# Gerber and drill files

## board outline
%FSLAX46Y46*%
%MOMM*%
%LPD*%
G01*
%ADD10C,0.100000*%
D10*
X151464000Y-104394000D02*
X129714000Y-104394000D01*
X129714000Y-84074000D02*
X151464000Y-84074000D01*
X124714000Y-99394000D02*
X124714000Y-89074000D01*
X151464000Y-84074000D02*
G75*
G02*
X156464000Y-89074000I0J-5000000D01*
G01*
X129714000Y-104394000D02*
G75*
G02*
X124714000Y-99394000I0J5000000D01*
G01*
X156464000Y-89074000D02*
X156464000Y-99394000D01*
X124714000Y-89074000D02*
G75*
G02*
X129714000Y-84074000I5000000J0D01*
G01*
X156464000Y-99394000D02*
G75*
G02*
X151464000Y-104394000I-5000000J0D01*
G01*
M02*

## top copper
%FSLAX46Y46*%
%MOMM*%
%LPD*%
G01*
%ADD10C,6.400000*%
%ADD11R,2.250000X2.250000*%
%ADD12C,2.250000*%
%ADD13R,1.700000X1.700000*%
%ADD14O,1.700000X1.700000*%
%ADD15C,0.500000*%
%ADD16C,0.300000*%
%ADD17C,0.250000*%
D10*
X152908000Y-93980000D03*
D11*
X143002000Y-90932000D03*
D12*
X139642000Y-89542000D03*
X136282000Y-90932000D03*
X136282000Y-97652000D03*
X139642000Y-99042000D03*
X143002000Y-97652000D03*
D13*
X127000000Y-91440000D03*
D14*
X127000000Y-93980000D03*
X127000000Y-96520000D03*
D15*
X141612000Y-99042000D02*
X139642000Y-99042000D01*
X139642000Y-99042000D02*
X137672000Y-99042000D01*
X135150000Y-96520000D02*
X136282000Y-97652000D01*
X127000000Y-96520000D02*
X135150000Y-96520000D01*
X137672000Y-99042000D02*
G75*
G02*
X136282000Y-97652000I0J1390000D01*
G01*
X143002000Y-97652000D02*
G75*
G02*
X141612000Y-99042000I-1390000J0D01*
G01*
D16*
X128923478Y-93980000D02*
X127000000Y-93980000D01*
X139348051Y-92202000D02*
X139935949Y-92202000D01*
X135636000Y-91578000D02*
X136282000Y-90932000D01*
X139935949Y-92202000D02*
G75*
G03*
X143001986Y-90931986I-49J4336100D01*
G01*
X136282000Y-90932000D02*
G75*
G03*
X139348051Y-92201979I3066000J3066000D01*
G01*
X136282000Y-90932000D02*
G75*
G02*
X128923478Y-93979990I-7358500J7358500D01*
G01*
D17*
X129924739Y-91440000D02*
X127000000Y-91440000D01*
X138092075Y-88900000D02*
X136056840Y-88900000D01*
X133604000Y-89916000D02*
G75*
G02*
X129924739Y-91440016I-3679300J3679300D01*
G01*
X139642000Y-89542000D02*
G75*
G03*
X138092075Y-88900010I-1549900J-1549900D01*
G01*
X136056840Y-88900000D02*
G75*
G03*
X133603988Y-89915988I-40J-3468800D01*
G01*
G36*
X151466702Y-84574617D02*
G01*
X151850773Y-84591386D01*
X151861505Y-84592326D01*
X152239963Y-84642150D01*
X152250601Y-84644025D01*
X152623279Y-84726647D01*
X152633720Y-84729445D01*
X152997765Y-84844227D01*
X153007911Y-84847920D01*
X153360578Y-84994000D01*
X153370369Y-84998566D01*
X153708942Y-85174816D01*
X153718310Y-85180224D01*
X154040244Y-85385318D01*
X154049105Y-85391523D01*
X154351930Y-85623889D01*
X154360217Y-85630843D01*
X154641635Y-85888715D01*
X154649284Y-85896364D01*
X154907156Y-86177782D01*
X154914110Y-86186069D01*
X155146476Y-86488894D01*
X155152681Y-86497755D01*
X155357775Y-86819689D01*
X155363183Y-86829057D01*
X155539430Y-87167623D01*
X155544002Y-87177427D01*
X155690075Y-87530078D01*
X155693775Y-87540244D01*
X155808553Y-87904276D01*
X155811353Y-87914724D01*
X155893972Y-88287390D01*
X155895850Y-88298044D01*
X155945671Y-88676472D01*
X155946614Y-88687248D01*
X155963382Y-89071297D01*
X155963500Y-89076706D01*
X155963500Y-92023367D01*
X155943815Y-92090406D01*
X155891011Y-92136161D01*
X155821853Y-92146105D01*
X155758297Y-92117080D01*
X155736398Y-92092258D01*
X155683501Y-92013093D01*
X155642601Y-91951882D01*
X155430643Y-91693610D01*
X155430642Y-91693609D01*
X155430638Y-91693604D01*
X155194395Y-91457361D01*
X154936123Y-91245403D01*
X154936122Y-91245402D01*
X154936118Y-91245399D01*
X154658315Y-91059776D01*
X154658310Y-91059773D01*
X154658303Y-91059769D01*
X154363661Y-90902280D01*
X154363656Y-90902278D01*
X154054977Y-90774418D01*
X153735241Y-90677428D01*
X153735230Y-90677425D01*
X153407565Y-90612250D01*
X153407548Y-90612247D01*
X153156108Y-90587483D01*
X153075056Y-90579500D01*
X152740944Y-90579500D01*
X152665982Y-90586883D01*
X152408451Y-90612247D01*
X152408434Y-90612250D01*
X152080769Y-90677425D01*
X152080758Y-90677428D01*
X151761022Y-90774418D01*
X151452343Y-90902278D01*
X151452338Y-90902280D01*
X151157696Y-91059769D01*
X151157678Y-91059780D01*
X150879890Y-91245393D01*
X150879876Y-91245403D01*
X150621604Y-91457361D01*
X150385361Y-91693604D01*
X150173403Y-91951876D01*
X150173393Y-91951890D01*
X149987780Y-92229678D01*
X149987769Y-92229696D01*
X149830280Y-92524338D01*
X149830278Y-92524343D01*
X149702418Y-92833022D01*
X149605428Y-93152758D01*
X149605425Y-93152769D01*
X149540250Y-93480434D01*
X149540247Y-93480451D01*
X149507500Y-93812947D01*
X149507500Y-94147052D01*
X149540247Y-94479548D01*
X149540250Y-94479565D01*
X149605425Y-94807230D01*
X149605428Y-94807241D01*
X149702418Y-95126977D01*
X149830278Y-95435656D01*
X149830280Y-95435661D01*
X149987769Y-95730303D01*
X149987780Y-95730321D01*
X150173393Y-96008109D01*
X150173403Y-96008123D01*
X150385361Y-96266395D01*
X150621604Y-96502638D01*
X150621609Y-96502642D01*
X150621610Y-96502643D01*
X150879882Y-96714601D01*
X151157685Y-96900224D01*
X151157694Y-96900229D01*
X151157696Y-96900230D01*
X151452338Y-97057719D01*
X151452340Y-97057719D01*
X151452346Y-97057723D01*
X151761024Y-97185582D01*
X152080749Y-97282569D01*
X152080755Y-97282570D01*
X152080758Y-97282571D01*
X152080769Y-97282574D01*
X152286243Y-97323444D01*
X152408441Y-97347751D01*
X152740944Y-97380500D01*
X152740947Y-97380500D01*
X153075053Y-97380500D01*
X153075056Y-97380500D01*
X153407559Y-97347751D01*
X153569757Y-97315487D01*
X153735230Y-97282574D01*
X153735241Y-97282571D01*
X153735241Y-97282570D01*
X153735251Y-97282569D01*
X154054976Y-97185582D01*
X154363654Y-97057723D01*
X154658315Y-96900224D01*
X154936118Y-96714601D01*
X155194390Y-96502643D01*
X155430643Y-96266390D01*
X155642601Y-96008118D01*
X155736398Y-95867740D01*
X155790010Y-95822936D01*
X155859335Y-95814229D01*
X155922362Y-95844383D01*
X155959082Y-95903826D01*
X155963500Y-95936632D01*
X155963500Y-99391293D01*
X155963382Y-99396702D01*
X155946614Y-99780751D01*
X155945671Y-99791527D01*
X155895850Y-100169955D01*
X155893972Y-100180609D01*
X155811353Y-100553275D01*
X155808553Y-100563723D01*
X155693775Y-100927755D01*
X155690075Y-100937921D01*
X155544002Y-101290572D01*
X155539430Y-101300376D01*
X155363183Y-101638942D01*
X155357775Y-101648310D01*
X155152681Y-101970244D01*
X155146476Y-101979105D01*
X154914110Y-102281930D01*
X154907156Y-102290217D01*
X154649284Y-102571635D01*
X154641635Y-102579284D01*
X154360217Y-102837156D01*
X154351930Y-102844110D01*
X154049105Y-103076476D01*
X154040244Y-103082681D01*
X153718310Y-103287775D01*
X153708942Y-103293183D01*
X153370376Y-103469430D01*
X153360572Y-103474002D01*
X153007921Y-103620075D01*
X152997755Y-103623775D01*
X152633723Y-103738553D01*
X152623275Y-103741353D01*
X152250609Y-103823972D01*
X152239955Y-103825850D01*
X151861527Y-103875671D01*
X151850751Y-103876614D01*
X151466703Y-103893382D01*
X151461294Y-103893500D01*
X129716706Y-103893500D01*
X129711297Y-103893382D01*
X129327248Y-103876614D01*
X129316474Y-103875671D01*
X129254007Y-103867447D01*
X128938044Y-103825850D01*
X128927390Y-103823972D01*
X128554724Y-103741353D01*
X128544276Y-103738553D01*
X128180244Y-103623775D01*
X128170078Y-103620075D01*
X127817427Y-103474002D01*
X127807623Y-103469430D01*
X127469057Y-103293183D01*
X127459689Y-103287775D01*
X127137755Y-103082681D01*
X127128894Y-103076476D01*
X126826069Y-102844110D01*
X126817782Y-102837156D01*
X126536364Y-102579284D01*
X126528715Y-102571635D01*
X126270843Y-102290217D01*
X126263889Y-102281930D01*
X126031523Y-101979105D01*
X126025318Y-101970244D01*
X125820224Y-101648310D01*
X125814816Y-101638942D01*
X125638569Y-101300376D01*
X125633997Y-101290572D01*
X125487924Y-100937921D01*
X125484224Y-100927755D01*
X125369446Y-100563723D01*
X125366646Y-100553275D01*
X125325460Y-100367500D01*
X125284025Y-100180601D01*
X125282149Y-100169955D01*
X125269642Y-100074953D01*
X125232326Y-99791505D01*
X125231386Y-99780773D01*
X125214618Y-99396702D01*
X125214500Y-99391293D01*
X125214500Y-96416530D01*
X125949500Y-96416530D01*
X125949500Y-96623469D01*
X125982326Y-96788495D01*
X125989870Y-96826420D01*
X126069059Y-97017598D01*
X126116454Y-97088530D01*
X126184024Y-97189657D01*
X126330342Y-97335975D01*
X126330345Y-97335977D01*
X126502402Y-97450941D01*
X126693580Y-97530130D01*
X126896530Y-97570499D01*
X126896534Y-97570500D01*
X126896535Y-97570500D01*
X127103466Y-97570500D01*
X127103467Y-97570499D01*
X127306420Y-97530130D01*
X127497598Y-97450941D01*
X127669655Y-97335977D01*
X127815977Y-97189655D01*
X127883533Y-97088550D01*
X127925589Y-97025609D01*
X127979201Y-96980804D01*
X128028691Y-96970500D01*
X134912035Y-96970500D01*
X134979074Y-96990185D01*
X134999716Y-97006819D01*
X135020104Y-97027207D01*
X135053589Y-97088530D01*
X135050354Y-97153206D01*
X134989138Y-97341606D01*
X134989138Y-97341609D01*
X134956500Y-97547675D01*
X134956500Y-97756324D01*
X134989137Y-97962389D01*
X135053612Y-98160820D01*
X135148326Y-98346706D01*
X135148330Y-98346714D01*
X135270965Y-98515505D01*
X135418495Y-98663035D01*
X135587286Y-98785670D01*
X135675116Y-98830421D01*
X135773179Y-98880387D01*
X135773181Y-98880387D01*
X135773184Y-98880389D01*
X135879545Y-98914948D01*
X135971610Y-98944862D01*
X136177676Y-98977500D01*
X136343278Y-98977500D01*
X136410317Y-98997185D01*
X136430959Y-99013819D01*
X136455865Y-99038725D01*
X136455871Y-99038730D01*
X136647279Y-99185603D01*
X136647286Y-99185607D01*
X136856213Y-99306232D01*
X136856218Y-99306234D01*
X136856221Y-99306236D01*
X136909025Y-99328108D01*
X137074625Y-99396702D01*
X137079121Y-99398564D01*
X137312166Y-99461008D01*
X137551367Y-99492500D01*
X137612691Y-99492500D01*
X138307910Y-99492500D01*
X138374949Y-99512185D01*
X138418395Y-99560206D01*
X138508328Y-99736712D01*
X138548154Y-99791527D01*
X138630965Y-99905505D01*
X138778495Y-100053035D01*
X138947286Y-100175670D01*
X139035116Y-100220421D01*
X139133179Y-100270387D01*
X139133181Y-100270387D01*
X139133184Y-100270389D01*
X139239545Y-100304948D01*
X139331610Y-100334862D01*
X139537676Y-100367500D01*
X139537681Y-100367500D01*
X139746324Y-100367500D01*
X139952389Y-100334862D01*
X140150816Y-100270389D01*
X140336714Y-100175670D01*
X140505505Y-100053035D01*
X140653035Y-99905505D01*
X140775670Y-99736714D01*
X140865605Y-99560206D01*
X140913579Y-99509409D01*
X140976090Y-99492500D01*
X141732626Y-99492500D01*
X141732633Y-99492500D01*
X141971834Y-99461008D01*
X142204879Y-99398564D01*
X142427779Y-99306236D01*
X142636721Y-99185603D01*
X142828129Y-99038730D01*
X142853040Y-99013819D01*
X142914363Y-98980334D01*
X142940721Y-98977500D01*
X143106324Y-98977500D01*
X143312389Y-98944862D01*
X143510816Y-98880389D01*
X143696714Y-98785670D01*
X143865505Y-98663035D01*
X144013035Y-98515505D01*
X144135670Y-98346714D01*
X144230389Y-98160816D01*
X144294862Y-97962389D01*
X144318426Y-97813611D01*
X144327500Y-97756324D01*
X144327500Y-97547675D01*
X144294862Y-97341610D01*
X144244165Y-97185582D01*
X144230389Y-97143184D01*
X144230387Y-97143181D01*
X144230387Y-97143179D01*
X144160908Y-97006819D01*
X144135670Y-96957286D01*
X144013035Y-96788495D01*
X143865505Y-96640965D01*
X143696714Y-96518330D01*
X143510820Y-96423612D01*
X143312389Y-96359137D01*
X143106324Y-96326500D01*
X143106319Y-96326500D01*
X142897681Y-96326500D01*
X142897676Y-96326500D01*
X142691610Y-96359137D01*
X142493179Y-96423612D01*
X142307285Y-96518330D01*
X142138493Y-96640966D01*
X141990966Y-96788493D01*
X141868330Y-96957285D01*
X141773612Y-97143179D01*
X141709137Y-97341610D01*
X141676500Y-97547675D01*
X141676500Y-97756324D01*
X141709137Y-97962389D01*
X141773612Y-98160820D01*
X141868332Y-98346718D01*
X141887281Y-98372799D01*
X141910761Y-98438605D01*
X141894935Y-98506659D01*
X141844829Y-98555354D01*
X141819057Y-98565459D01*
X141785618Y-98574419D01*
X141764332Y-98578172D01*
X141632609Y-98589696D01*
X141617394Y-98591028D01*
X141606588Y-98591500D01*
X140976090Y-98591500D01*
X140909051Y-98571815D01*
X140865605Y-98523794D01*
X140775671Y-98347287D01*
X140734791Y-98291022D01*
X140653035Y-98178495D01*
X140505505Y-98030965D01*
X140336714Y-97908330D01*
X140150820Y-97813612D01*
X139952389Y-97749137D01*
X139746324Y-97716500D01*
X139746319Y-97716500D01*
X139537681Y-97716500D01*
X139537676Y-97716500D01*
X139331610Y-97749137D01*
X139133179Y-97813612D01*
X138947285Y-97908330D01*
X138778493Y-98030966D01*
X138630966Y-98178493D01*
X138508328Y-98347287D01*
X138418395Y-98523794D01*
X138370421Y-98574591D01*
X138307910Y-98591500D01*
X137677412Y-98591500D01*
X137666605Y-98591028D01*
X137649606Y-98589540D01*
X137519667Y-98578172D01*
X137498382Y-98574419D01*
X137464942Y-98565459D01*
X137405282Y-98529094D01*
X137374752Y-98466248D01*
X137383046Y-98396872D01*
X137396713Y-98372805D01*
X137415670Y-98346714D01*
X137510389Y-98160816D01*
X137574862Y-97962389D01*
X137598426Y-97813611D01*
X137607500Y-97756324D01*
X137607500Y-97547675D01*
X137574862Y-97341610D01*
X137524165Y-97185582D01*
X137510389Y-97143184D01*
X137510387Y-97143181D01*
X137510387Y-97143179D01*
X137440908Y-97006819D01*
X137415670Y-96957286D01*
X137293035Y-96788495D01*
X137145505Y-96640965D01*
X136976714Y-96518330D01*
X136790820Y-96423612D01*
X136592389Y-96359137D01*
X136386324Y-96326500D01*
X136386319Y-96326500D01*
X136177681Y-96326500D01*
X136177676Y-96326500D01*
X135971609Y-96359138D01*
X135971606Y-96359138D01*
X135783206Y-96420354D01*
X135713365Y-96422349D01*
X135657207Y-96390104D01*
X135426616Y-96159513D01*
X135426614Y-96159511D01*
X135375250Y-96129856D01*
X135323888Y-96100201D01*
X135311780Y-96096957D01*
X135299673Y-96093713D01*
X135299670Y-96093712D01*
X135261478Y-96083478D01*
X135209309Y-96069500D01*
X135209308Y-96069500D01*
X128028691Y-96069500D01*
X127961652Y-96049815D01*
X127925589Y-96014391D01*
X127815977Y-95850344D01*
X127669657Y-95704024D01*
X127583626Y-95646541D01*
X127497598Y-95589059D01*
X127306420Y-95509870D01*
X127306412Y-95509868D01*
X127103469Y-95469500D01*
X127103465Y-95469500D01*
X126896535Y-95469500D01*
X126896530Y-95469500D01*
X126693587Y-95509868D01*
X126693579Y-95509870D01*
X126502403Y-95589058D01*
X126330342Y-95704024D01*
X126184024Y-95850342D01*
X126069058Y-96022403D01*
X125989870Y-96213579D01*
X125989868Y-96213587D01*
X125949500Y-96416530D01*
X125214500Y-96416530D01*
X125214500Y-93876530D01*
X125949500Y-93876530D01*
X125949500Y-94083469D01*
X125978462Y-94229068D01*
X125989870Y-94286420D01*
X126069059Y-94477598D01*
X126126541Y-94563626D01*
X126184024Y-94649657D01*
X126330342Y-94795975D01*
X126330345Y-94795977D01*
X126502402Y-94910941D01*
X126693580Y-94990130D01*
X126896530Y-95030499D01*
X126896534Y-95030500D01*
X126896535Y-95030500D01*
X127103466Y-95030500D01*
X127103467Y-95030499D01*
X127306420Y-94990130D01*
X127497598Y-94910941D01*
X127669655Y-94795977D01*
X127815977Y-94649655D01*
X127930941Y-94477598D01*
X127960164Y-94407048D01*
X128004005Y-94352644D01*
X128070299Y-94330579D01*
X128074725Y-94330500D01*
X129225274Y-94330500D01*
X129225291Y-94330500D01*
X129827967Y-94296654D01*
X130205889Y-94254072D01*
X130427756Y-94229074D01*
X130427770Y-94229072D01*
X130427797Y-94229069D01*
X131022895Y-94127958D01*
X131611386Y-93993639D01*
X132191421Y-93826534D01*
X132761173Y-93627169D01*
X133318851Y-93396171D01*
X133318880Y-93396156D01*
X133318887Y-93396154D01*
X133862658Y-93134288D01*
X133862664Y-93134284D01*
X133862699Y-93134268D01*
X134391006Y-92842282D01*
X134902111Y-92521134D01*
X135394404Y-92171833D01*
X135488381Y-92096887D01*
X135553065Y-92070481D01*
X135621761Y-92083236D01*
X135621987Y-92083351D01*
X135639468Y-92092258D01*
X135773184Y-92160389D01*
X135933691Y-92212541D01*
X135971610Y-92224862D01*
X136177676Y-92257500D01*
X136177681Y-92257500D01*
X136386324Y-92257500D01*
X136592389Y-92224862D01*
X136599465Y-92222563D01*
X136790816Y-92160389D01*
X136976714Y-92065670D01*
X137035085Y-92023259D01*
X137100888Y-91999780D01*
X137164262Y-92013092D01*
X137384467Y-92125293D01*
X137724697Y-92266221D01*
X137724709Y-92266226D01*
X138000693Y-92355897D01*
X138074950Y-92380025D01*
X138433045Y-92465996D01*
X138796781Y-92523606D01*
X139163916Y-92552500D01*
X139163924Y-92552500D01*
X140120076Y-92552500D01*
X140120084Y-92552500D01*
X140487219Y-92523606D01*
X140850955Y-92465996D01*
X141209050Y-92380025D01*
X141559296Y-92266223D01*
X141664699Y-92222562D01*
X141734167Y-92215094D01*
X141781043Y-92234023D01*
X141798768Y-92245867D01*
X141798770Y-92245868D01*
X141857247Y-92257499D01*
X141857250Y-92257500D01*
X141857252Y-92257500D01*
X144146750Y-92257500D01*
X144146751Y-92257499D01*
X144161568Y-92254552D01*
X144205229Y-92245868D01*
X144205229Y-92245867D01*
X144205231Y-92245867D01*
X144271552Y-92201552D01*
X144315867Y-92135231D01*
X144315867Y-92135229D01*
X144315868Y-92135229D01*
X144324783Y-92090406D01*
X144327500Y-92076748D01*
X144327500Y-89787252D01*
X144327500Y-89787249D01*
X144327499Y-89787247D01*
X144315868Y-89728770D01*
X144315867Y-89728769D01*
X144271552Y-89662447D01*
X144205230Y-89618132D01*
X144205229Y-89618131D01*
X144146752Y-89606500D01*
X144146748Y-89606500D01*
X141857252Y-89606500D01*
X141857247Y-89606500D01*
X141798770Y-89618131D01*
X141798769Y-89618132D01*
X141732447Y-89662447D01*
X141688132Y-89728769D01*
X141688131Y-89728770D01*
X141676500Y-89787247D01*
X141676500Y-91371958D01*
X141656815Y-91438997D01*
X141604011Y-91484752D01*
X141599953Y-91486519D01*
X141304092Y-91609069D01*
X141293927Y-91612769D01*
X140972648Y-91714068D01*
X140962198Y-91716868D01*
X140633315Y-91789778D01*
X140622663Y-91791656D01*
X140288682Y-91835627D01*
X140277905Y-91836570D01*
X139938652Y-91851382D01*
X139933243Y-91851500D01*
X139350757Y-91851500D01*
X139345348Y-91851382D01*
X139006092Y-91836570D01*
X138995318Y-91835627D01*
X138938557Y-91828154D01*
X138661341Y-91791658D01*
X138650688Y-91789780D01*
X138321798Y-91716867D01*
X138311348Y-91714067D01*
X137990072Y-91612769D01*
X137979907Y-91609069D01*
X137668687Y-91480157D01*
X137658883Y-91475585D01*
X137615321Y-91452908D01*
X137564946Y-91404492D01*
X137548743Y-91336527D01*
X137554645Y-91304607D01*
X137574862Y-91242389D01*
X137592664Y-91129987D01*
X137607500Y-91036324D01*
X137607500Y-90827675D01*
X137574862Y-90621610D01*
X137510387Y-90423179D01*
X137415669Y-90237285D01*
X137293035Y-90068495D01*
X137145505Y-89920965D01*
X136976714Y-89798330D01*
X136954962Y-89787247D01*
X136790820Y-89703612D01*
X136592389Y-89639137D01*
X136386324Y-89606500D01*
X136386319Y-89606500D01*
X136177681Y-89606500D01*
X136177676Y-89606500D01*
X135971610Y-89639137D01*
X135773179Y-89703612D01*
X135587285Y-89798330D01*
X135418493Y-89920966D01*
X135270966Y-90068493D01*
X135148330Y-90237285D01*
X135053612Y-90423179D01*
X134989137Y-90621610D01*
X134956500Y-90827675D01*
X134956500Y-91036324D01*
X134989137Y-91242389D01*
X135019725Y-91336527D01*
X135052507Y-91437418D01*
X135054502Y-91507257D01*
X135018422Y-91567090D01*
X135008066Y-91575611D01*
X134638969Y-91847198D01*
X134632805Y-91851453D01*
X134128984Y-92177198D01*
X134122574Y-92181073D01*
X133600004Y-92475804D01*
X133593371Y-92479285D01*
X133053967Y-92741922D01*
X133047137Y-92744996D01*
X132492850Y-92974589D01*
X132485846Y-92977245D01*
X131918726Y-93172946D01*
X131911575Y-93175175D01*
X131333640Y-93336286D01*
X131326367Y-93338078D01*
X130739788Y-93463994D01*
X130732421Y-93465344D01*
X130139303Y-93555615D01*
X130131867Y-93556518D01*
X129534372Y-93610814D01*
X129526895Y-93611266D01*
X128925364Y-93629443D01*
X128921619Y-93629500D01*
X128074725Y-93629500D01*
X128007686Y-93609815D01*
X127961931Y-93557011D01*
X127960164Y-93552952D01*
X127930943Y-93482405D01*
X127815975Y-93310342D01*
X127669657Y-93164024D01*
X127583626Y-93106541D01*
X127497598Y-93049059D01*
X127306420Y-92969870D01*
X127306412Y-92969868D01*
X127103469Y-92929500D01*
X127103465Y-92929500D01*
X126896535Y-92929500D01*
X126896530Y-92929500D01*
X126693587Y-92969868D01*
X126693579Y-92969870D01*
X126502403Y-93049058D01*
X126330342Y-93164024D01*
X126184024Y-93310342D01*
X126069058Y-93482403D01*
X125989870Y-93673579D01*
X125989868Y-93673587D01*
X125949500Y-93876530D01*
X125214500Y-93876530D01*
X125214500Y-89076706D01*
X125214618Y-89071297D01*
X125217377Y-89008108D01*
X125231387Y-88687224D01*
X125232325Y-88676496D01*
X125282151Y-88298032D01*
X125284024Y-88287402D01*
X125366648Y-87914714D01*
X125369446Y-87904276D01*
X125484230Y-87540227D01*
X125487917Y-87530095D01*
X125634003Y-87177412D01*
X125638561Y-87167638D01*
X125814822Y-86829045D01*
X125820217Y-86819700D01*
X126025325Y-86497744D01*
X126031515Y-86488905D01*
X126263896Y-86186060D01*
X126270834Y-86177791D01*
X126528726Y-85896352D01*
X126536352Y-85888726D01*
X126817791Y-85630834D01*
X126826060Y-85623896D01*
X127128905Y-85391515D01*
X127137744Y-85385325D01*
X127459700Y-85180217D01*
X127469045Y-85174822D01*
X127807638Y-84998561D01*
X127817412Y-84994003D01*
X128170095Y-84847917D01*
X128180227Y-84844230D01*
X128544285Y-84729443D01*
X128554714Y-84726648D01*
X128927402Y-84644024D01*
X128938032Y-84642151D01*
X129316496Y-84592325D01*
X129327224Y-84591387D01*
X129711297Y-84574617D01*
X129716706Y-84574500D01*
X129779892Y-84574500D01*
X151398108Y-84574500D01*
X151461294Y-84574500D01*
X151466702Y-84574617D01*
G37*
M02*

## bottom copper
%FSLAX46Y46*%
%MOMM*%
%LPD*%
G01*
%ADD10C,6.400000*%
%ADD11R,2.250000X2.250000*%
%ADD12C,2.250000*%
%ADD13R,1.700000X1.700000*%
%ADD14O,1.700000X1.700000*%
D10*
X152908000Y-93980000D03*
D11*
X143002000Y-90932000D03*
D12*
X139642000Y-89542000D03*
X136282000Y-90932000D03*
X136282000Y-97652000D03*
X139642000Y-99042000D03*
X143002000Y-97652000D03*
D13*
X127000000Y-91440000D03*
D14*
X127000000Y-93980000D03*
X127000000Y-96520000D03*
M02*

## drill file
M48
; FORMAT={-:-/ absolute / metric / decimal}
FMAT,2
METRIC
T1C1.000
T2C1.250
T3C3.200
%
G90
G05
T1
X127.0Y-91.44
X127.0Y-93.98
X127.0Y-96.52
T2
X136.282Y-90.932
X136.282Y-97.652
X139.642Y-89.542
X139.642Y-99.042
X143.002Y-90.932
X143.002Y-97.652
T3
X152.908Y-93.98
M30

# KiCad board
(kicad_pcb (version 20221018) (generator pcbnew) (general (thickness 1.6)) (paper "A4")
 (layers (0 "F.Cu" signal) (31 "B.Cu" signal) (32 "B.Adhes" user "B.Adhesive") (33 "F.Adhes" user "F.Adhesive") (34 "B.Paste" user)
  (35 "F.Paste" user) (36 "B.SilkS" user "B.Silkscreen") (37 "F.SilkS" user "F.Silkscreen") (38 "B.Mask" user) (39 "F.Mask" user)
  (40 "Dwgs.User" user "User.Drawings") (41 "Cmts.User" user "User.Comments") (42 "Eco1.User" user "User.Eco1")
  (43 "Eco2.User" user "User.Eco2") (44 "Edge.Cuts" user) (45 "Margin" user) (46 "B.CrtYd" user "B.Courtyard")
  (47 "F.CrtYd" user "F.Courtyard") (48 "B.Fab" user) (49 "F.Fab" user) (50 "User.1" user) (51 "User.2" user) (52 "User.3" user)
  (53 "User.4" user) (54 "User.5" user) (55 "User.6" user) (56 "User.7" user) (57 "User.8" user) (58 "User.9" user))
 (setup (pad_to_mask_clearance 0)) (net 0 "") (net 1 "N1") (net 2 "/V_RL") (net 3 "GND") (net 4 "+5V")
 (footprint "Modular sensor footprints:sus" (layer "F.Cu") (at 139.642 94.292)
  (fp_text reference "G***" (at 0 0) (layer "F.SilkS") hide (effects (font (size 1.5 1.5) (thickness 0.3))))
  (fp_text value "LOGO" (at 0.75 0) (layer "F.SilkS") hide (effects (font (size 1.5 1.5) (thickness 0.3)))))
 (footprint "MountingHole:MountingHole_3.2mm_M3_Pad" (layer "F.Cu") (at 152.908 93.98)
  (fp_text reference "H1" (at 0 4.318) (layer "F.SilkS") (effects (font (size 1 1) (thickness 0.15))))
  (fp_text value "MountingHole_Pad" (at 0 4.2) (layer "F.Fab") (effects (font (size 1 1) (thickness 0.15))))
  (pad "1" thru_hole circle (at 0 0) (size 6.4 6.4) (drill 3.2) (layers "*.Cu" "*.Mask") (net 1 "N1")))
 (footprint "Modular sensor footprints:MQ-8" (layer "F.Cu") (at 143.002 90.932 -90)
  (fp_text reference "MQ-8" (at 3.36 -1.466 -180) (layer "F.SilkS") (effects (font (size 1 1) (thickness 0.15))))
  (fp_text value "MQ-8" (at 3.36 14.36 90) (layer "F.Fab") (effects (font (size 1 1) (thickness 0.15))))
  (pad "1" thru_hole rect (at 0 0 270) (size 2.25 2.25) (drill 1.25) (layers "*.Cu" "*.Mask") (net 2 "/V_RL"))
  (pad "2" thru_hole circle (at -1.39 3.36 270) (size 2.25 2.25) (drill 1.25) (layers "*.Cu" "*.Mask") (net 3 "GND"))
  (pad "3" thru_hole circle (at 0 6.72) (size 2.25 2.25) (drill 1.25) (layers "*.Cu" "*.Mask") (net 2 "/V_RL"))
  (pad "4" thru_hole circle (at 6.72 6.72 90) (size 2.25 2.25) (drill 1.25) (layers "*.Cu" "*.Mask") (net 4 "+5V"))
  (pad "5" thru_hole circle (at 8.11 3.36 270) (size 2.25 2.25) (drill 1.25) (layers "*.Cu" "*.Mask") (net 4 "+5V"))
  (pad "6" thru_hole circle (at 6.72 0 180) (size 2.25 2.25) (drill 1.25) (layers "*.Cu" "*.Mask") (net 4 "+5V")))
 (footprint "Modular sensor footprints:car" (layer "B.Cu") (at 144.018 86.614 180)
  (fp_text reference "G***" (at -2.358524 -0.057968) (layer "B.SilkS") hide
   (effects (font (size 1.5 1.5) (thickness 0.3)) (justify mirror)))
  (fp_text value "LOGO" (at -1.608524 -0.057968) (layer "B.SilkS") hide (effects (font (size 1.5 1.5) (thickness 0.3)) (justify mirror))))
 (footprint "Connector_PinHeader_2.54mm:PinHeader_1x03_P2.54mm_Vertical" (layer "B.Cu") (at 127 91.44 180)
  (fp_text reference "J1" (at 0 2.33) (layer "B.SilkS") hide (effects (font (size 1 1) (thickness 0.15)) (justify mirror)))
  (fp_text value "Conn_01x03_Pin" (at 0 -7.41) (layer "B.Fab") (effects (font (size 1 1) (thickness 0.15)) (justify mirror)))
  (pad "1" thru_hole rect (at 0 0 180) (size 1.7 1.7) (drill 1) (layers "*.Cu" "*.Mask") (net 3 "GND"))
  (pad "2" thru_hole oval (at 0 -2.54 180) (size 1.7 1.7) (drill 1) (layers "*.Cu" "*.Mask") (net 2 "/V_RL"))
  (pad "3" thru_hole oval (at 0 -5.08 180) (size 1.7 1.7) (drill 1) (layers "*.Cu" "*.Mask") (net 4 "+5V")))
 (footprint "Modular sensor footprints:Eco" (layer "B.Cu") (at 146.535078 86.615892 180)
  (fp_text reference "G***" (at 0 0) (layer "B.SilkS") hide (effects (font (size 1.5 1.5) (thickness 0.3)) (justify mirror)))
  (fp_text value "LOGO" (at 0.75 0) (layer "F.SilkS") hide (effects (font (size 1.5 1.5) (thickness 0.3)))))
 (gr_line (start 151.464 104.394) (end 129.714 104.394) (stroke (width 0.1) (type default)) (layer "Edge.Cuts"))
 (gr_line (start 129.714 84.074) (end 151.464 84.074) (stroke (width 0.1) (type default)) (layer "Edge.Cuts"))
 (gr_line (start 124.714 99.394) (end 124.714 89.074) (stroke (width 0.1) (type default)) (layer "Edge.Cuts"))
 (gr_arc (start 151.464 84.074) (mid 154.999534 85.538466) (end 156.464 89.074) (stroke (width 0.1) (type default)) (layer "Edge.Cuts"))
 (gr_arc (start 129.714 104.394) (mid 126.178466 102.929534) (end 124.714 99.394) (stroke (width 0.1) (type default)) (layer "Edge.Cuts"))
 (gr_line (start 156.464 89.074) (end 156.464 99.394) (stroke (width 0.1) (type default)) (layer "Edge.Cuts"))
 (gr_arc (start 124.714 89.074) (mid 126.178466 85.538466) (end 129.714 84.074) (stroke (width 0.1) (type default)) (layer "Edge.Cuts"))
 (gr_arc (start 156.464 99.394) (mid 154.999534 102.929534) (end 151.464 104.394) (stroke (width 0.1) (type default)) (layer "Edge.Cuts"))
 (segment (start 141.612 99.042) (end 139.642 99.042) (width 0.5) (layer "F.Cu") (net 4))
 (segment (start 139.642 99.042) (end 137.672 99.042) (width 0.5) (layer "F.Cu") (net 4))
 (segment (start 135.15 96.52) (end 136.282 97.652) (width 0.5) (layer "F.Cu") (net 4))
 (segment (start 127 96.52) (end 135.15 96.52) (width 0.5) (layer "F.Cu") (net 4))
 (arc (start 137.672 99.042) (mid 136.689122 98.634878) (end 136.282 97.652) (width 0.5) (layer "F.Cu") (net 4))
 (arc (start 143.002 97.652) (mid 142.594878 98.634878) (end 141.612 99.042) (width 0.5) (layer "F.Cu") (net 4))
 (segment (start 128.923478 93.98) (end 127 93.98) (width 0.3) (layer "F.Cu") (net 2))
 (segment (start 139.348051 92.202) (end 139.935949 92.202) (width 0.3) (layer "F.Cu") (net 2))
 (segment (start 135.636 91.578) (end 136.282 90.932) (width 0.3) (layer "F.Cu") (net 2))
 (arc (start 139.935949 92.202) (mid 141.595283 91.871938) (end 143.002 90.932) (width 0.3) (layer "F.Cu") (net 2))
 (arc (start 136.282 90.932) (mid 137.688715 91.871938) (end 139.348051 92.202) (width 0.3) (layer "F.Cu") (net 2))
 (arc (start 136.282 90.932) (mid 132.905882 93.18785) (end 128.923478 93.98) (width 0.3) (layer "F.Cu") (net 2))
 (segment (start 129.924739 91.44) (end 127 91.44) (width 0.25) (layer "F.Cu") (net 3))
 (segment (start 138.092075 88.9) (end 136.05684 88.9) (width 0.25) (layer "F.Cu") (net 3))
 (arc (start 133.604 89.916) (mid 131.915941 91.043925) (end 129.924739 91.44) (width 0.25) (layer "F.Cu") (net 3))
 (arc (start 139.642 89.542) (mid 138.930889 89.06685) (end 138.092075 88.9) (width 0.25) (layer "F.Cu") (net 3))
 (arc (start 136.05684 88.9) (mid 134.729372 89.16405) (end 133.604 89.916) (width 0.25) (layer "F.Cu") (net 3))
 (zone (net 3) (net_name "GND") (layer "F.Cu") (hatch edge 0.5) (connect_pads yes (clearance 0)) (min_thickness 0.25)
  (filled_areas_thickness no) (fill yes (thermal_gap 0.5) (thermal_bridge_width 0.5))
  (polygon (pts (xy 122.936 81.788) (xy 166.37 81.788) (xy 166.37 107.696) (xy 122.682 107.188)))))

